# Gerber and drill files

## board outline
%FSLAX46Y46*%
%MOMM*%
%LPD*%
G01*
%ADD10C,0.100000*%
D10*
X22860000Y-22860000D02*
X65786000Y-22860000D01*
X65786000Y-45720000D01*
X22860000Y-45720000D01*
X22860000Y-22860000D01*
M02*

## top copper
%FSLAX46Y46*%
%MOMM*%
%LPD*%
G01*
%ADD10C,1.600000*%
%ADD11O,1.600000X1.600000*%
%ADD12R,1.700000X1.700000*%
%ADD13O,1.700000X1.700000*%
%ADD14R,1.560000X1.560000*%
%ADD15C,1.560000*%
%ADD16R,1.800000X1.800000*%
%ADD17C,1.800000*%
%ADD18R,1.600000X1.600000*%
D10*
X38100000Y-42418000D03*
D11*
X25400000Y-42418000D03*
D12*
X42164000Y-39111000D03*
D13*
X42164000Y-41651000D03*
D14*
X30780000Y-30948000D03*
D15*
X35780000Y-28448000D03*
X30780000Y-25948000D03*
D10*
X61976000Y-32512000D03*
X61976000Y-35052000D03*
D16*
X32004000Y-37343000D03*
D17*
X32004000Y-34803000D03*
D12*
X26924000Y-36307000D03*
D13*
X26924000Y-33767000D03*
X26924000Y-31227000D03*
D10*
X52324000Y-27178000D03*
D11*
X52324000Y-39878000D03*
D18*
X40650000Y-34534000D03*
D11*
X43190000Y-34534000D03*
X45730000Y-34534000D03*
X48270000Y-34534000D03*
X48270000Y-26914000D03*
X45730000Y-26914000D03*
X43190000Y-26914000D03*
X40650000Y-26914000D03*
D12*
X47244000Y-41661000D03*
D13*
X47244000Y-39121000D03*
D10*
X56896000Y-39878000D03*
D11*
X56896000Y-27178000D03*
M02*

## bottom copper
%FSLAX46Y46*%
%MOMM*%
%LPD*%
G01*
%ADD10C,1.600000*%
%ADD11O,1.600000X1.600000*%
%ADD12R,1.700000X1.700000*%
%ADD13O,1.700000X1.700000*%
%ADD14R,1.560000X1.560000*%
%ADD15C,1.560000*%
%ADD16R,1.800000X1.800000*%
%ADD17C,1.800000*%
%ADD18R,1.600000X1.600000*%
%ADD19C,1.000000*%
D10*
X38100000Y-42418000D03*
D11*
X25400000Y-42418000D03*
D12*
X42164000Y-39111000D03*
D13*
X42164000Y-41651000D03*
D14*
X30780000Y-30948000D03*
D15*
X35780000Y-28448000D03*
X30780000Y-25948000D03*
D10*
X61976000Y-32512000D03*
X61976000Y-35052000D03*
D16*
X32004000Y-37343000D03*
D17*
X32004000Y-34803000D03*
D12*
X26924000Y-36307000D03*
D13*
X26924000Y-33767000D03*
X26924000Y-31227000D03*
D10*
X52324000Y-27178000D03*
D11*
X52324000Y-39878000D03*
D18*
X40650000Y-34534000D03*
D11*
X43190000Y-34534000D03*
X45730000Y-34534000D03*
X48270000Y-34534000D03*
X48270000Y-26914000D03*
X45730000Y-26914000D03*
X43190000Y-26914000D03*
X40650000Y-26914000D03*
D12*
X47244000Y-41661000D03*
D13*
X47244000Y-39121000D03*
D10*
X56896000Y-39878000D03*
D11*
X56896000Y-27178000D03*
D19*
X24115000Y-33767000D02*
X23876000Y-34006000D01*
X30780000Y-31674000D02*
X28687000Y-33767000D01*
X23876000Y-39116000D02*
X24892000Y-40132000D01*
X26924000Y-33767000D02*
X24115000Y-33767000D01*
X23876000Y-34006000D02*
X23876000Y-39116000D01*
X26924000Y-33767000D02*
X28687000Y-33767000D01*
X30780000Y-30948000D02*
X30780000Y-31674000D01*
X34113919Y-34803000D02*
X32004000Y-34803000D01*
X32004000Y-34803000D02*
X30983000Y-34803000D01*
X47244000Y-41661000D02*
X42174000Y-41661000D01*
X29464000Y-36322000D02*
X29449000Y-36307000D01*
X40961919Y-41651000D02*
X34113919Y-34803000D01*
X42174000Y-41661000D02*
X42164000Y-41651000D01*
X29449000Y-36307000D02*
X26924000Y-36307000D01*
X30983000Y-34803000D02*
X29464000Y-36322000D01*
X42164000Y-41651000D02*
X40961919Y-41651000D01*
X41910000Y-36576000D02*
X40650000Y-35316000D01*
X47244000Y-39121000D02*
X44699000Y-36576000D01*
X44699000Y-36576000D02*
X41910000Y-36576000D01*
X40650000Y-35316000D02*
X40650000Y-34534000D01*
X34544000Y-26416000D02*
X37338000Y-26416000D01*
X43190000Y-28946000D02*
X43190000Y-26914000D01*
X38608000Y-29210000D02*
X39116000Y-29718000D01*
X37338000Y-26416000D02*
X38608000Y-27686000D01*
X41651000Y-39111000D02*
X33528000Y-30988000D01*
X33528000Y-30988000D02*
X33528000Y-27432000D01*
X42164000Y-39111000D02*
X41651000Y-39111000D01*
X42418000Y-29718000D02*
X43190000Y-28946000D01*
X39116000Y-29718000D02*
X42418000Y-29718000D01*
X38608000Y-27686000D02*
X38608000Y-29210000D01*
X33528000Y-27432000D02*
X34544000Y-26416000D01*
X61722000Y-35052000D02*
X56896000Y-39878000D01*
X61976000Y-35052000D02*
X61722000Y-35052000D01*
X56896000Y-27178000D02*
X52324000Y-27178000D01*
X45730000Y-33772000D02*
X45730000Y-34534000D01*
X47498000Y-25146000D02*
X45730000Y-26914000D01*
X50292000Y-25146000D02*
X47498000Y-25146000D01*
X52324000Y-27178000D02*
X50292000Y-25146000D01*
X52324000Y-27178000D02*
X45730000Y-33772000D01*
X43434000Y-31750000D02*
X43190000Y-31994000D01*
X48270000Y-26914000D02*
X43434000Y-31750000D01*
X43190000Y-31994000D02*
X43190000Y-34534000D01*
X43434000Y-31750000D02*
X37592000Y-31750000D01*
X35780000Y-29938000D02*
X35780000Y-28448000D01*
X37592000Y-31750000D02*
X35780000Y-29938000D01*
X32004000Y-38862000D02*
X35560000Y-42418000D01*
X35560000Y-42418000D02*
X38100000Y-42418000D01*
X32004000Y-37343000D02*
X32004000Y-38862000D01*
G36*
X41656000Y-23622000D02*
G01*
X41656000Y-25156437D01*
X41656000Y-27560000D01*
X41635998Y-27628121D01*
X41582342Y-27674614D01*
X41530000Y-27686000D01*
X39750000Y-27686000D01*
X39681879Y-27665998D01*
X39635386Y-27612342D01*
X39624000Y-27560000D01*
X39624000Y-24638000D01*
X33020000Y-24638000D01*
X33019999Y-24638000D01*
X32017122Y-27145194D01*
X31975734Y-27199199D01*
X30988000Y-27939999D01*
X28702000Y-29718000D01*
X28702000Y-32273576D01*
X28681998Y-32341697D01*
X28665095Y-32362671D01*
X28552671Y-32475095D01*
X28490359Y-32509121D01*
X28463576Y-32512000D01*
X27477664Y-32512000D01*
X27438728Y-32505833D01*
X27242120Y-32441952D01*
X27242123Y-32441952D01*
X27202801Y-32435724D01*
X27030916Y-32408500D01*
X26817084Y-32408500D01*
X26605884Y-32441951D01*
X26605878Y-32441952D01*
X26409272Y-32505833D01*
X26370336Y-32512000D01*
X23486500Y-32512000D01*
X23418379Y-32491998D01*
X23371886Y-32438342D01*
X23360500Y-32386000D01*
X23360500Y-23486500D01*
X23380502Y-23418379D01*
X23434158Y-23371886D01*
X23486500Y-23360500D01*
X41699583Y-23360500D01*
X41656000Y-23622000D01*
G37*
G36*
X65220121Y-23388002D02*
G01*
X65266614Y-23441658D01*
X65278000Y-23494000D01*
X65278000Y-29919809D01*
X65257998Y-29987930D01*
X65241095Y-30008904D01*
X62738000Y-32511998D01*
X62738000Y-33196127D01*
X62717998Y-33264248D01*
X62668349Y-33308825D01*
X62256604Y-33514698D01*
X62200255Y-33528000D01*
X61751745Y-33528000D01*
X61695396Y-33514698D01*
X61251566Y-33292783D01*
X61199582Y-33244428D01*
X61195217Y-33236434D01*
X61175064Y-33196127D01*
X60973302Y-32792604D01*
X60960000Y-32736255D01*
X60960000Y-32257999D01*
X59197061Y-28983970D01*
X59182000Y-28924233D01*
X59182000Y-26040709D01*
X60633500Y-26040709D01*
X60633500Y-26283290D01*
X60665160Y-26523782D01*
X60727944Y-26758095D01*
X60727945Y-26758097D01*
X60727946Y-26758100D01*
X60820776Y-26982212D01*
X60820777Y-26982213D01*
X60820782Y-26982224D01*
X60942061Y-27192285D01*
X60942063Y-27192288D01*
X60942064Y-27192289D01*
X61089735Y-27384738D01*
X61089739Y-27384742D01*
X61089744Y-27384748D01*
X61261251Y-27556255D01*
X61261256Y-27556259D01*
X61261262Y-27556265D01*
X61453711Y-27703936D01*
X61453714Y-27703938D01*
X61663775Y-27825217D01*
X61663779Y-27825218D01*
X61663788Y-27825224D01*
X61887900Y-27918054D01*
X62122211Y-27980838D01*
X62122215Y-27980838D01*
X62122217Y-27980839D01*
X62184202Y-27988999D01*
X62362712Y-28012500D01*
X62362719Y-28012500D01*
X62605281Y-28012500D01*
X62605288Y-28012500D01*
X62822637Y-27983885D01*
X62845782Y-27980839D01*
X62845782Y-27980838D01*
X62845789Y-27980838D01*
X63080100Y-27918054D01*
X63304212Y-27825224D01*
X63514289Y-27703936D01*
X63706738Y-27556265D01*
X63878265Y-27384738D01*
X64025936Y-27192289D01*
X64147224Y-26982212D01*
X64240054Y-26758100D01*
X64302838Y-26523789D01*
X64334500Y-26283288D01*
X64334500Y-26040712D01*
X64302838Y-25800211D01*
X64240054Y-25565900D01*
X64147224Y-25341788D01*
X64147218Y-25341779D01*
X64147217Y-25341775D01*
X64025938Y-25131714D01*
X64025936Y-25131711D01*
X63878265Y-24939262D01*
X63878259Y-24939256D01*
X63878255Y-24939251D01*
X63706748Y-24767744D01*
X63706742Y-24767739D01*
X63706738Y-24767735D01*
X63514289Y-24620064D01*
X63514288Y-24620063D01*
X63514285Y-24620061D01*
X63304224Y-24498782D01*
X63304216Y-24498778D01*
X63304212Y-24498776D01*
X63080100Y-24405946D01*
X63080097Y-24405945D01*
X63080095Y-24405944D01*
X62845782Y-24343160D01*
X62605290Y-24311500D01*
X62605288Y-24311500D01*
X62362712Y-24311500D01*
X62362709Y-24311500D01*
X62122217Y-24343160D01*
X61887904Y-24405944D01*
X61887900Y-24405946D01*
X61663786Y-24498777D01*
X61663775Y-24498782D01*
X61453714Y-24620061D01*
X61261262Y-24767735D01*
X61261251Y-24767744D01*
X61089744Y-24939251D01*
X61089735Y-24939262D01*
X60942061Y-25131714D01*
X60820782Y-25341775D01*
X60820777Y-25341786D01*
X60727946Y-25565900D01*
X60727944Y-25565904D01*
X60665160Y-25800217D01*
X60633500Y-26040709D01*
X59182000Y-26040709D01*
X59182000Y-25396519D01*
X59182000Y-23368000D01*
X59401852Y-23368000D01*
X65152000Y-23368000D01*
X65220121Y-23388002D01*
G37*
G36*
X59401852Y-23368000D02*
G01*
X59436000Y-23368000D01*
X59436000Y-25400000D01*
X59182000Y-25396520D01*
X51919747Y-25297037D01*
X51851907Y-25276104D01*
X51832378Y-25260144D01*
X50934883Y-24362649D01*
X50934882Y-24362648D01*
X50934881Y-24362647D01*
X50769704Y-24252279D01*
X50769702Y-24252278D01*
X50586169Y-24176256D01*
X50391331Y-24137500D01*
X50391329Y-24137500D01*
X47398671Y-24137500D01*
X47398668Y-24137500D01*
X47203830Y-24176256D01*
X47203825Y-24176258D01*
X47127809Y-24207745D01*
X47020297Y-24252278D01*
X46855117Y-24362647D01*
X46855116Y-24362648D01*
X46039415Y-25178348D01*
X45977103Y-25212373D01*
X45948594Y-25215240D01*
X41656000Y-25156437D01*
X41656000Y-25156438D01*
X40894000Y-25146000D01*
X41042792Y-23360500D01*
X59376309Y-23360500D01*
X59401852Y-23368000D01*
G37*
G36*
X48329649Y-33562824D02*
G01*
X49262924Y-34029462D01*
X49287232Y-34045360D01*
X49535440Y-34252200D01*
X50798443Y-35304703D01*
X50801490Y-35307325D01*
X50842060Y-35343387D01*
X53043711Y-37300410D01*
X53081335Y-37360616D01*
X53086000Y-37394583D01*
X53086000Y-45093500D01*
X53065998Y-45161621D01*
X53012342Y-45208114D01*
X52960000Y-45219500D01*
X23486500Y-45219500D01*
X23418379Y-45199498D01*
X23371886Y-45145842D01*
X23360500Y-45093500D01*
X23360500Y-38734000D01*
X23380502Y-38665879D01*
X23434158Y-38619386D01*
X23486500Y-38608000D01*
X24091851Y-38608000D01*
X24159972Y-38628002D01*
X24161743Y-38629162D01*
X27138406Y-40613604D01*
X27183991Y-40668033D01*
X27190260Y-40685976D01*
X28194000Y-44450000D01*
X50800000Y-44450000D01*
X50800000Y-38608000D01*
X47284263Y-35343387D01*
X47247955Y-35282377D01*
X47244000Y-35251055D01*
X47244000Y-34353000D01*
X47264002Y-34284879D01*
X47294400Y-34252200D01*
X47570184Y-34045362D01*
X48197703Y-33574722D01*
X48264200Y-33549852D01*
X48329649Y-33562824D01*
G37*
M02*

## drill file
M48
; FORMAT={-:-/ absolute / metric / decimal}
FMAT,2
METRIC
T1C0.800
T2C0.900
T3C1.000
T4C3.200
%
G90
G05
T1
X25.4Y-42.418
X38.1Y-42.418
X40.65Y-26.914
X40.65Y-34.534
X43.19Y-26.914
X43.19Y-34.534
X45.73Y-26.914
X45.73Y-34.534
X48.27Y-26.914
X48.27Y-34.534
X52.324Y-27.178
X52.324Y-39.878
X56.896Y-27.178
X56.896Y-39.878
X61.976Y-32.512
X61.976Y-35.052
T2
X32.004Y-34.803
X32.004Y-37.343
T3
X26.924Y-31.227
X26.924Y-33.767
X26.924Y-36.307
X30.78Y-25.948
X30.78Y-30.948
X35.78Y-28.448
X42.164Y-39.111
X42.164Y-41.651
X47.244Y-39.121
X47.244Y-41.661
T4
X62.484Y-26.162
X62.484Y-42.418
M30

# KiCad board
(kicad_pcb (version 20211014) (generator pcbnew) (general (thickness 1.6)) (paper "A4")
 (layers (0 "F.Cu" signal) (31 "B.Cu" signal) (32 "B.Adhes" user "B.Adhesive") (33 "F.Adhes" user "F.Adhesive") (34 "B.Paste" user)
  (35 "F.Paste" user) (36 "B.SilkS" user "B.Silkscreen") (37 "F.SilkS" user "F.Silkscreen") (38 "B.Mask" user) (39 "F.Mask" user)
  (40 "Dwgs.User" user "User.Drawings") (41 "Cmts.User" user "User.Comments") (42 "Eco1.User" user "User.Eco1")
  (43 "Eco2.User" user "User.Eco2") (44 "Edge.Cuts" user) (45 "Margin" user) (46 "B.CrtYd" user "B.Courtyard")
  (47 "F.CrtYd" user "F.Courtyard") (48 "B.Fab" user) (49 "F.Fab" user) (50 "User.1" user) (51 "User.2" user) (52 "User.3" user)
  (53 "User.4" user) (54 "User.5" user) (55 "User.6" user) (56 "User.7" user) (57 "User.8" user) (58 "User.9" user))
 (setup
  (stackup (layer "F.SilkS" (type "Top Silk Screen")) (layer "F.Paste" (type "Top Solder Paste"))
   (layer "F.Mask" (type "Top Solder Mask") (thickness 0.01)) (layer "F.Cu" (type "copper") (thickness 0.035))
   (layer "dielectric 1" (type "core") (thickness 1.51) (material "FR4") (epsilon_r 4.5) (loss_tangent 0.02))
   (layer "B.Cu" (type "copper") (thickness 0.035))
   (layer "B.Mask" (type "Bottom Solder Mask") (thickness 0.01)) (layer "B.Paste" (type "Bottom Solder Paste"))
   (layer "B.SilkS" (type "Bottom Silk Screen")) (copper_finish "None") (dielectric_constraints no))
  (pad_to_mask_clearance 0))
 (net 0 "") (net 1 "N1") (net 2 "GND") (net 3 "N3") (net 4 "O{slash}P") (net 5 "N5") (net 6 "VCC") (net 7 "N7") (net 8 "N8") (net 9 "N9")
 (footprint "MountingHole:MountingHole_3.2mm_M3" (layer "F.Cu") (at 62.484 42.418)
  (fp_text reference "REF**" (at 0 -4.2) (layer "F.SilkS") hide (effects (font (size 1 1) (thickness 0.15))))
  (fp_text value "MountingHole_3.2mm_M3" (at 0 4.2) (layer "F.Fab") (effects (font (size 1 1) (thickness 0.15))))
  (pad "" np_thru_hole circle locked (at 0 0) (size 3.2 3.2) (drill 3.2) (layers F&B.Cu *.Mask)))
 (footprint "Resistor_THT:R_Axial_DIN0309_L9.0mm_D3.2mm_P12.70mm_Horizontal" (layer "F.Cu") (at 38.1 42.418 180)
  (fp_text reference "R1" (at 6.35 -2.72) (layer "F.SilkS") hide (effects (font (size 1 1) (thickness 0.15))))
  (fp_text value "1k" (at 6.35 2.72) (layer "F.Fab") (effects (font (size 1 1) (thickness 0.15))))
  (pad "1" thru_hole circle (at 0 0 180) (size 1.6 1.6) (drill 0.8) (layers *.Cu *.Mask) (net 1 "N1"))
  (pad "2" thru_hole oval (at 12.7 0 180) (size 1.6 1.6) (drill 0.8) (layers *.Cu *.Mask) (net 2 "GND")))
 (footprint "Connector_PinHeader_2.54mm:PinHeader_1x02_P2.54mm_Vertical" (layer "F.Cu") (at 42.164 39.111)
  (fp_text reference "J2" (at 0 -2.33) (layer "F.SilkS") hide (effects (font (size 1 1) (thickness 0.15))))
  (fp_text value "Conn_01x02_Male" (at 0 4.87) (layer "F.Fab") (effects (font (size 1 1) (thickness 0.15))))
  (pad "1" thru_hole rect (at 0 0) (size 1.7 1.7) (drill 1) (layers *.Cu *.Mask) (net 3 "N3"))
  (pad "2" thru_hole oval (at 0 2.54) (size 1.7 1.7) (drill 1) (layers *.Cu *.Mask) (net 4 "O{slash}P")))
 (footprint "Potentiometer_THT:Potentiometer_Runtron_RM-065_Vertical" (layer "F.Cu") (at 30.78 30.948 90)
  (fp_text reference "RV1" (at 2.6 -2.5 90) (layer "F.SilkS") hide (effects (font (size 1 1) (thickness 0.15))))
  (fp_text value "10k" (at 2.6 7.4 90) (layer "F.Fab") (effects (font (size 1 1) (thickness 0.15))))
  (pad "1" thru_hole rect (at 0 0 90) (size 1.56 1.56) (drill 1) (layers *.Cu *.Mask) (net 2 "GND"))
  (pad "2" thru_hole circle (at 2.5 5 90) (size 1.56 1.56) (drill 1) (layers *.Cu *.Mask) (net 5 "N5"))
  (pad "3" thru_hole circle (at 5 0 90) (size 1.56 1.56) (drill 1) (layers *.Cu *.Mask) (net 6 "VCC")))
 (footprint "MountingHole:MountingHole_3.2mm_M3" (layer "F.Cu") (at 62.484 26.162)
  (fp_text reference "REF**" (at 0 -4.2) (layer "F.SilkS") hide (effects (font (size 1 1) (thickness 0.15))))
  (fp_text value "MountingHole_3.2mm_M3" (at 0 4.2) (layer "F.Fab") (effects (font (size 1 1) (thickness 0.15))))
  (pad "" np_thru_hole circle locked (at 0 0) (size 3.2 3.2) (drill 3.2) (layers F&B.Cu *.Mask)))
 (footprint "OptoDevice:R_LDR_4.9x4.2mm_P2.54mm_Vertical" (layer "F.Cu") (at 61.976 32.512 -90)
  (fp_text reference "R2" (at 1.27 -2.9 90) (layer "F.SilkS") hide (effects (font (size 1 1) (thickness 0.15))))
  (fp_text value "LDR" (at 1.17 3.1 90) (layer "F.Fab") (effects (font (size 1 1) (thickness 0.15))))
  (pad "1" thru_hole circle (at 0 0 270) (size 1.6 1.6) (drill 0.8) (layers *.Cu *.Mask) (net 6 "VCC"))
  (pad "2" thru_hole circle (at 2.54 0 270) (size 1.6 1.6) (drill 0.8) (layers *.Cu *.Mask) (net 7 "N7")))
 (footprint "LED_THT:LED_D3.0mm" (layer "F.Cu") (at 32.004 37.343 90)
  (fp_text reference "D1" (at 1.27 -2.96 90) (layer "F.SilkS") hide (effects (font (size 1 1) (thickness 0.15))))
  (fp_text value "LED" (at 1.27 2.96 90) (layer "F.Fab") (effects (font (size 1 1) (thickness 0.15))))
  (pad "1" thru_hole rect (at 0 0 90) (size 1.8 1.8) (drill 0.9) (layers *.Cu *.Mask) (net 1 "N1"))
  (pad "2" thru_hole circle (at 2.54 0 90) (size 1.8 1.8) (drill 0.9) (layers *.Cu *.Mask) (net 4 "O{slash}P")))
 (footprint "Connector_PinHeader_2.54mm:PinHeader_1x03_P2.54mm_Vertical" (layer "F.Cu") (at 26.924 36.307 180)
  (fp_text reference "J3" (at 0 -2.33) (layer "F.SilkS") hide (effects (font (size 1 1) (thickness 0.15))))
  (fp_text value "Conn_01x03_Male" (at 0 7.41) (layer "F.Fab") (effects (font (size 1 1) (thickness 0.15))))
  (pad "1" thru_hole rect (at 0 0 180) (size 1.7 1.7) (drill 1) (layers *.Cu *.Mask) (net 4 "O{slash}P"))
  (pad "2" thru_hole oval (at 0 2.54 180) (size 1.7 1.7) (drill 1) (layers *.Cu *.Mask) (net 2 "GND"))
  (pad "3" thru_hole oval (at 0 5.08 180) (size 1.7 1.7) (drill 1) (layers *.Cu *.Mask) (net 6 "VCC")))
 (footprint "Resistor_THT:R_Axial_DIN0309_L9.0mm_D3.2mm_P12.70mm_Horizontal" (layer "F.Cu") (at 52.324 27.178 -90)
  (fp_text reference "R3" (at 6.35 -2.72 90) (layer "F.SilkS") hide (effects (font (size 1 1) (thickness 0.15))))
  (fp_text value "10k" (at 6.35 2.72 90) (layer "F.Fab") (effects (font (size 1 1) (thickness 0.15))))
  (pad "1" thru_hole circle (at 0 0 270) (size 1.6 1.6) (drill 0.8) (layers *.Cu *.Mask) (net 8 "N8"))
  (pad "2" thru_hole oval (at 12.7 0 270) (size 1.6 1.6) (drill 0.8) (layers *.Cu *.Mask) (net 2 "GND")))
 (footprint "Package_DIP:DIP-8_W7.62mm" (layer "F.Cu") (at 40.65 34.534 90)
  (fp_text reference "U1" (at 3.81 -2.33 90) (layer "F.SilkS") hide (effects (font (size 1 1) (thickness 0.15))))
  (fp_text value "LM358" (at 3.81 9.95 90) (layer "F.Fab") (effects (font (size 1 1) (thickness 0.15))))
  (pad "1" thru_hole rect (at 0 0 90) (size 1.6 1.6) (drill 0.8) (layers *.Cu *.Mask) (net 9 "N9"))
  (pad "2" thru_hole oval (at 0 2.54 90) (size 1.6 1.6) (drill 0.8) (layers *.Cu *.Mask) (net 5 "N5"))
  (pad "3" thru_hole oval (at 0 5.08 90) (size 1.6 1.6) (drill 0.8) (layers *.Cu *.Mask) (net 8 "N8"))
  (pad "4" thru_hole oval (at 0 7.62 90) (size 1.6 1.6) (drill 0.8) (layers *.Cu *.Mask) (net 2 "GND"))
  (pad "5" thru_hole oval (at 7.62 7.62 90) (size 1.6 1.6) (drill 0.8) (layers *.Cu *.Mask) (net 5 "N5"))
  (pad "6" thru_hole oval (at 7.62 5.08 90) (size 1.6 1.6) (drill 0.8) (layers *.Cu *.Mask) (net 8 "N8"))
  (pad "7" thru_hole oval (at 7.62 2.54 90) (size 1.6 1.6) (drill 0.8) (layers *.Cu *.Mask) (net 3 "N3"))
  (pad "8" thru_hole oval (at 7.62 0 90) (size 1.6 1.6) (drill 0.8) (layers *.Cu *.Mask) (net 6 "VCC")))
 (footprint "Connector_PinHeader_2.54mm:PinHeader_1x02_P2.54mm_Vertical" (layer "F.Cu") (at 47.244 41.661 180)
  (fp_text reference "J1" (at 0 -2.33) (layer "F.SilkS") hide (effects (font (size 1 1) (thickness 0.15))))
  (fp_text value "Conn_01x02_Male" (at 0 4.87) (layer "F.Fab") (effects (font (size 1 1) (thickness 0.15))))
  (pad "1" thru_hole rect (at 0 0 180) (size 1.7 1.7) (drill 1) (layers *.Cu *.Mask) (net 4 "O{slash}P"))
  (pad "2" thru_hole oval (at 0 2.54 180) (size 1.7 1.7) (drill 1) (layers *.Cu *.Mask) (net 9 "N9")))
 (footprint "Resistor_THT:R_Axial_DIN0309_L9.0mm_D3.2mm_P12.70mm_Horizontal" (layer "F.Cu") (at 56.896 39.878 90)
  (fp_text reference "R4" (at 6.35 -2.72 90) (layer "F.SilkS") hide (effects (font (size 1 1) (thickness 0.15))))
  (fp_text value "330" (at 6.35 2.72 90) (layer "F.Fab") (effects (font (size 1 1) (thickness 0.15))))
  (pad "1" thru_hole circle (at 0 0 90) (size 1.6 1.6) (drill 0.8) (layers *.Cu *.Mask) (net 7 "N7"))
  (pad "2" thru_hole oval (at 12.7 0 90) (size 1.6 1.6) (drill 0.8) (layers *.Cu *.Mask) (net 8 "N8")))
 (gr_rect (start 22.86 22.86) (end 65.786 45.72) (layer "Edge.Cuts") (width 0.1) (fill none))
 (segment (start 24.115 33.767) (end 23.876 34.006) (width 1) (layer "B.Cu") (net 2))
 (segment (start 30.78 31.674) (end 28.687 33.767) (width 1) (layer "B.Cu") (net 2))
 (segment (start 23.876 39.116) (end 24.892 40.132) (width 1) (layer "B.Cu") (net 2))
 (segment (start 26.924 33.767) (end 24.115 33.767) (width 1) (layer "B.Cu") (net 2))
 (segment (start 23.876 34.006) (end 23.876 39.116) (width 1) (layer "B.Cu") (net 2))
 (segment (start 26.924 33.767) (end 28.687 33.767) (width 1) (layer "B.Cu") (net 2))
 (segment (start 30.78 30.948) (end 30.78 31.674) (width 1) (layer "B.Cu") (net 2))
 (segment (start 34.113919 34.803) (end 32.004 34.803) (width 1) (layer "B.Cu") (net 4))
 (segment (start 32.004 34.803) (end 30.983 34.803) (width 1) (layer "B.Cu") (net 4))
 (segment (start 47.244 41.661) (end 42.174 41.661) (width 1) (layer "B.Cu") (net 4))
 (segment (start 29.464 36.322) (end 29.449 36.307) (width 1) (layer "B.Cu") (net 4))
 (segment (start 40.961919 41.651) (end 34.113919 34.803) (width 1) (layer "B.Cu") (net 4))
 (segment (start 42.174 41.661) (end 42.164 41.651) (width 1) (layer "B.Cu") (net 4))
 (segment (start 29.449 36.307) (end 26.924 36.307) (width 1) (layer "B.Cu") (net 4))
 (segment (start 30.983 34.803) (end 29.464 36.322) (width 1) (layer "B.Cu") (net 4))
 (segment (start 42.164 41.651) (end 40.961919 41.651) (width 1) (layer "B.Cu") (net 4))
 (segment (start 41.91 36.576) (end 40.65 35.316) (width 1) (layer "B.Cu") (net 9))
 (segment (start 47.244 39.121) (end 44.699 36.576) (width 1) (layer "B.Cu") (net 9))
 (segment (start 44.699 36.576) (end 41.91 36.576) (width 1) (layer "B.Cu") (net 9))
 (segment (start 40.65 35.316) (end 40.65 34.534) (width 1) (layer "B.Cu") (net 9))
 (segment (start 34.544 26.416) (end 37.338 26.416) (width 1) (layer "B.Cu") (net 3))
 (segment (start 43.19 28.946) (end 43.19 26.914) (width 1) (layer "B.Cu") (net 3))
 (segment (start 38.608 29.21) (end 39.116 29.718) (width 1) (layer "B.Cu") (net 3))
 (segment (start 37.338 26.416) (end 38.608 27.686) (width 1) (layer "B.Cu") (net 3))
 (segment (start 41.651 39.111) (end 33.528 30.988) (width 1) (layer "B.Cu") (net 3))
 (segment (start 33.528 30.988) (end 33.528 27.432) (width 1) (layer "B.Cu") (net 3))
 (segment (start 42.164 39.111) (end 41.651 39.111) (width 1) (layer "B.Cu") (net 3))
 (segment (start 42.418 29.718) (end 43.19 28.946) (width 1) (layer "B.Cu") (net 3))
 (segment (start 39.116 29.718) (end 42.418 29.718) (width 1) (layer "B.Cu") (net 3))
 (segment (start 38.608 27.686) (end 38.608 29.21) (width 1) (layer "B.Cu") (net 3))
 (segment (start 33.528 27.432) (end 34.544 26.416) (width 1) (layer "B.Cu") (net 3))
 (segment (start 61.722 35.052) (end 56.896 39.878) (width 1) (layer "B.Cu") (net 7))
 (segment (start 61.976 35.052) (end 61.722 35.052) (width 1) (layer "B.Cu") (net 7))
 (segment (start 56.896 27.178) (end 52.324 27.178) (width 1) (layer "B.Cu") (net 8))
 (segment (start 45.73 33.772) (end 45.73 34.534) (width 1) (layer "B.Cu") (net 8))
 (segment (start 47.498 25.146) (end 45.73 26.914) (width 1) (layer "B.Cu") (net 8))
 (segment (start 50.292 25.146) (end 47.498 25.146) (width 1) (layer "B.Cu") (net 8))
 (segment (start 52.324 27.178) (end 50.292 25.146) (width 1) (layer "B.Cu") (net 8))
 (segment (start 52.324 27.178) (end 45.73 33.772) (width 1) (layer "B.Cu") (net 8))
 (segment (start 43.434 31.75) (end 43.19 31.994) (width 1) (layer "B.Cu") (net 5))
 (segment (start 48.27 26.914) (end 43.434 31.75) (width 1) (layer "B.Cu") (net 5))
 (segment (start 43.19 31.994) (end 43.19 34.534) (width 1) (layer "B.Cu") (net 5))
 (segment (start 43.434 31.75) (end 37.592 31.75) (width 1) (layer "B.Cu") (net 5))
 (segment (start 35.78 29.938) (end 35.78 28.448) (width 1) (layer "B.Cu") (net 5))
 (segment (start 37.592 31.75) (end 35.78 29.938) (width 1) (layer "B.Cu") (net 5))
 (segment (start 32.004 38.862) (end 35.56 42.418) (width 1) (layer "B.Cu") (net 1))
 (segment (start 35.56 42.418) (end 38.1 42.418) (width 1) (layer "B.Cu") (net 1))
 (segment (start 32.004 37.343) (end 32.004 38.862) (width 1) (layer "B.Cu") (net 1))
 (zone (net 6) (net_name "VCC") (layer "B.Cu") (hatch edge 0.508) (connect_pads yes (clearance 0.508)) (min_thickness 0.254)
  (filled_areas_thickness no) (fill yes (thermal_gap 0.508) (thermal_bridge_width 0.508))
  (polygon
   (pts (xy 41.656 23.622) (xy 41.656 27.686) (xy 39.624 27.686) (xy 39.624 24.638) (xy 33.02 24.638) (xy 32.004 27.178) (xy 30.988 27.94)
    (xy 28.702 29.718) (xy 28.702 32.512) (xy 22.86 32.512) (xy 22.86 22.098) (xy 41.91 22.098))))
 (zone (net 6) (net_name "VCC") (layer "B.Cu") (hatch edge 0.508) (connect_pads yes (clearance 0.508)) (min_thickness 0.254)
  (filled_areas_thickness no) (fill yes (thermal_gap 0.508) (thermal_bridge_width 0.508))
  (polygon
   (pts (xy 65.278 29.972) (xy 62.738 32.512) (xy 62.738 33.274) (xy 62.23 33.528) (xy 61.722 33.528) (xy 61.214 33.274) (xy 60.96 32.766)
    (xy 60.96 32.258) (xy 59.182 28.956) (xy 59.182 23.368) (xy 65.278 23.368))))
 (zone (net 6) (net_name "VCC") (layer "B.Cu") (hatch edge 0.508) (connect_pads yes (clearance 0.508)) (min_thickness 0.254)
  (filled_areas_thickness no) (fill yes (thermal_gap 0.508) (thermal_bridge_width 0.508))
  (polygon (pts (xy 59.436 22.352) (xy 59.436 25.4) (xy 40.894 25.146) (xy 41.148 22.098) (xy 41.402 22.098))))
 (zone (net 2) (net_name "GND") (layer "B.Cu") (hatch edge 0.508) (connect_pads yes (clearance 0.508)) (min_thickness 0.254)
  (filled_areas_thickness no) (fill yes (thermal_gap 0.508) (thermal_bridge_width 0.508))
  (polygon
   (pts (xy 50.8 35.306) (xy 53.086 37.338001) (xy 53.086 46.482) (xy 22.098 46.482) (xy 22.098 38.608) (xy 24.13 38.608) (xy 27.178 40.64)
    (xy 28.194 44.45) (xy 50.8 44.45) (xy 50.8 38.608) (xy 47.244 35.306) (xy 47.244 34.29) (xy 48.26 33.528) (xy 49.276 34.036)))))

